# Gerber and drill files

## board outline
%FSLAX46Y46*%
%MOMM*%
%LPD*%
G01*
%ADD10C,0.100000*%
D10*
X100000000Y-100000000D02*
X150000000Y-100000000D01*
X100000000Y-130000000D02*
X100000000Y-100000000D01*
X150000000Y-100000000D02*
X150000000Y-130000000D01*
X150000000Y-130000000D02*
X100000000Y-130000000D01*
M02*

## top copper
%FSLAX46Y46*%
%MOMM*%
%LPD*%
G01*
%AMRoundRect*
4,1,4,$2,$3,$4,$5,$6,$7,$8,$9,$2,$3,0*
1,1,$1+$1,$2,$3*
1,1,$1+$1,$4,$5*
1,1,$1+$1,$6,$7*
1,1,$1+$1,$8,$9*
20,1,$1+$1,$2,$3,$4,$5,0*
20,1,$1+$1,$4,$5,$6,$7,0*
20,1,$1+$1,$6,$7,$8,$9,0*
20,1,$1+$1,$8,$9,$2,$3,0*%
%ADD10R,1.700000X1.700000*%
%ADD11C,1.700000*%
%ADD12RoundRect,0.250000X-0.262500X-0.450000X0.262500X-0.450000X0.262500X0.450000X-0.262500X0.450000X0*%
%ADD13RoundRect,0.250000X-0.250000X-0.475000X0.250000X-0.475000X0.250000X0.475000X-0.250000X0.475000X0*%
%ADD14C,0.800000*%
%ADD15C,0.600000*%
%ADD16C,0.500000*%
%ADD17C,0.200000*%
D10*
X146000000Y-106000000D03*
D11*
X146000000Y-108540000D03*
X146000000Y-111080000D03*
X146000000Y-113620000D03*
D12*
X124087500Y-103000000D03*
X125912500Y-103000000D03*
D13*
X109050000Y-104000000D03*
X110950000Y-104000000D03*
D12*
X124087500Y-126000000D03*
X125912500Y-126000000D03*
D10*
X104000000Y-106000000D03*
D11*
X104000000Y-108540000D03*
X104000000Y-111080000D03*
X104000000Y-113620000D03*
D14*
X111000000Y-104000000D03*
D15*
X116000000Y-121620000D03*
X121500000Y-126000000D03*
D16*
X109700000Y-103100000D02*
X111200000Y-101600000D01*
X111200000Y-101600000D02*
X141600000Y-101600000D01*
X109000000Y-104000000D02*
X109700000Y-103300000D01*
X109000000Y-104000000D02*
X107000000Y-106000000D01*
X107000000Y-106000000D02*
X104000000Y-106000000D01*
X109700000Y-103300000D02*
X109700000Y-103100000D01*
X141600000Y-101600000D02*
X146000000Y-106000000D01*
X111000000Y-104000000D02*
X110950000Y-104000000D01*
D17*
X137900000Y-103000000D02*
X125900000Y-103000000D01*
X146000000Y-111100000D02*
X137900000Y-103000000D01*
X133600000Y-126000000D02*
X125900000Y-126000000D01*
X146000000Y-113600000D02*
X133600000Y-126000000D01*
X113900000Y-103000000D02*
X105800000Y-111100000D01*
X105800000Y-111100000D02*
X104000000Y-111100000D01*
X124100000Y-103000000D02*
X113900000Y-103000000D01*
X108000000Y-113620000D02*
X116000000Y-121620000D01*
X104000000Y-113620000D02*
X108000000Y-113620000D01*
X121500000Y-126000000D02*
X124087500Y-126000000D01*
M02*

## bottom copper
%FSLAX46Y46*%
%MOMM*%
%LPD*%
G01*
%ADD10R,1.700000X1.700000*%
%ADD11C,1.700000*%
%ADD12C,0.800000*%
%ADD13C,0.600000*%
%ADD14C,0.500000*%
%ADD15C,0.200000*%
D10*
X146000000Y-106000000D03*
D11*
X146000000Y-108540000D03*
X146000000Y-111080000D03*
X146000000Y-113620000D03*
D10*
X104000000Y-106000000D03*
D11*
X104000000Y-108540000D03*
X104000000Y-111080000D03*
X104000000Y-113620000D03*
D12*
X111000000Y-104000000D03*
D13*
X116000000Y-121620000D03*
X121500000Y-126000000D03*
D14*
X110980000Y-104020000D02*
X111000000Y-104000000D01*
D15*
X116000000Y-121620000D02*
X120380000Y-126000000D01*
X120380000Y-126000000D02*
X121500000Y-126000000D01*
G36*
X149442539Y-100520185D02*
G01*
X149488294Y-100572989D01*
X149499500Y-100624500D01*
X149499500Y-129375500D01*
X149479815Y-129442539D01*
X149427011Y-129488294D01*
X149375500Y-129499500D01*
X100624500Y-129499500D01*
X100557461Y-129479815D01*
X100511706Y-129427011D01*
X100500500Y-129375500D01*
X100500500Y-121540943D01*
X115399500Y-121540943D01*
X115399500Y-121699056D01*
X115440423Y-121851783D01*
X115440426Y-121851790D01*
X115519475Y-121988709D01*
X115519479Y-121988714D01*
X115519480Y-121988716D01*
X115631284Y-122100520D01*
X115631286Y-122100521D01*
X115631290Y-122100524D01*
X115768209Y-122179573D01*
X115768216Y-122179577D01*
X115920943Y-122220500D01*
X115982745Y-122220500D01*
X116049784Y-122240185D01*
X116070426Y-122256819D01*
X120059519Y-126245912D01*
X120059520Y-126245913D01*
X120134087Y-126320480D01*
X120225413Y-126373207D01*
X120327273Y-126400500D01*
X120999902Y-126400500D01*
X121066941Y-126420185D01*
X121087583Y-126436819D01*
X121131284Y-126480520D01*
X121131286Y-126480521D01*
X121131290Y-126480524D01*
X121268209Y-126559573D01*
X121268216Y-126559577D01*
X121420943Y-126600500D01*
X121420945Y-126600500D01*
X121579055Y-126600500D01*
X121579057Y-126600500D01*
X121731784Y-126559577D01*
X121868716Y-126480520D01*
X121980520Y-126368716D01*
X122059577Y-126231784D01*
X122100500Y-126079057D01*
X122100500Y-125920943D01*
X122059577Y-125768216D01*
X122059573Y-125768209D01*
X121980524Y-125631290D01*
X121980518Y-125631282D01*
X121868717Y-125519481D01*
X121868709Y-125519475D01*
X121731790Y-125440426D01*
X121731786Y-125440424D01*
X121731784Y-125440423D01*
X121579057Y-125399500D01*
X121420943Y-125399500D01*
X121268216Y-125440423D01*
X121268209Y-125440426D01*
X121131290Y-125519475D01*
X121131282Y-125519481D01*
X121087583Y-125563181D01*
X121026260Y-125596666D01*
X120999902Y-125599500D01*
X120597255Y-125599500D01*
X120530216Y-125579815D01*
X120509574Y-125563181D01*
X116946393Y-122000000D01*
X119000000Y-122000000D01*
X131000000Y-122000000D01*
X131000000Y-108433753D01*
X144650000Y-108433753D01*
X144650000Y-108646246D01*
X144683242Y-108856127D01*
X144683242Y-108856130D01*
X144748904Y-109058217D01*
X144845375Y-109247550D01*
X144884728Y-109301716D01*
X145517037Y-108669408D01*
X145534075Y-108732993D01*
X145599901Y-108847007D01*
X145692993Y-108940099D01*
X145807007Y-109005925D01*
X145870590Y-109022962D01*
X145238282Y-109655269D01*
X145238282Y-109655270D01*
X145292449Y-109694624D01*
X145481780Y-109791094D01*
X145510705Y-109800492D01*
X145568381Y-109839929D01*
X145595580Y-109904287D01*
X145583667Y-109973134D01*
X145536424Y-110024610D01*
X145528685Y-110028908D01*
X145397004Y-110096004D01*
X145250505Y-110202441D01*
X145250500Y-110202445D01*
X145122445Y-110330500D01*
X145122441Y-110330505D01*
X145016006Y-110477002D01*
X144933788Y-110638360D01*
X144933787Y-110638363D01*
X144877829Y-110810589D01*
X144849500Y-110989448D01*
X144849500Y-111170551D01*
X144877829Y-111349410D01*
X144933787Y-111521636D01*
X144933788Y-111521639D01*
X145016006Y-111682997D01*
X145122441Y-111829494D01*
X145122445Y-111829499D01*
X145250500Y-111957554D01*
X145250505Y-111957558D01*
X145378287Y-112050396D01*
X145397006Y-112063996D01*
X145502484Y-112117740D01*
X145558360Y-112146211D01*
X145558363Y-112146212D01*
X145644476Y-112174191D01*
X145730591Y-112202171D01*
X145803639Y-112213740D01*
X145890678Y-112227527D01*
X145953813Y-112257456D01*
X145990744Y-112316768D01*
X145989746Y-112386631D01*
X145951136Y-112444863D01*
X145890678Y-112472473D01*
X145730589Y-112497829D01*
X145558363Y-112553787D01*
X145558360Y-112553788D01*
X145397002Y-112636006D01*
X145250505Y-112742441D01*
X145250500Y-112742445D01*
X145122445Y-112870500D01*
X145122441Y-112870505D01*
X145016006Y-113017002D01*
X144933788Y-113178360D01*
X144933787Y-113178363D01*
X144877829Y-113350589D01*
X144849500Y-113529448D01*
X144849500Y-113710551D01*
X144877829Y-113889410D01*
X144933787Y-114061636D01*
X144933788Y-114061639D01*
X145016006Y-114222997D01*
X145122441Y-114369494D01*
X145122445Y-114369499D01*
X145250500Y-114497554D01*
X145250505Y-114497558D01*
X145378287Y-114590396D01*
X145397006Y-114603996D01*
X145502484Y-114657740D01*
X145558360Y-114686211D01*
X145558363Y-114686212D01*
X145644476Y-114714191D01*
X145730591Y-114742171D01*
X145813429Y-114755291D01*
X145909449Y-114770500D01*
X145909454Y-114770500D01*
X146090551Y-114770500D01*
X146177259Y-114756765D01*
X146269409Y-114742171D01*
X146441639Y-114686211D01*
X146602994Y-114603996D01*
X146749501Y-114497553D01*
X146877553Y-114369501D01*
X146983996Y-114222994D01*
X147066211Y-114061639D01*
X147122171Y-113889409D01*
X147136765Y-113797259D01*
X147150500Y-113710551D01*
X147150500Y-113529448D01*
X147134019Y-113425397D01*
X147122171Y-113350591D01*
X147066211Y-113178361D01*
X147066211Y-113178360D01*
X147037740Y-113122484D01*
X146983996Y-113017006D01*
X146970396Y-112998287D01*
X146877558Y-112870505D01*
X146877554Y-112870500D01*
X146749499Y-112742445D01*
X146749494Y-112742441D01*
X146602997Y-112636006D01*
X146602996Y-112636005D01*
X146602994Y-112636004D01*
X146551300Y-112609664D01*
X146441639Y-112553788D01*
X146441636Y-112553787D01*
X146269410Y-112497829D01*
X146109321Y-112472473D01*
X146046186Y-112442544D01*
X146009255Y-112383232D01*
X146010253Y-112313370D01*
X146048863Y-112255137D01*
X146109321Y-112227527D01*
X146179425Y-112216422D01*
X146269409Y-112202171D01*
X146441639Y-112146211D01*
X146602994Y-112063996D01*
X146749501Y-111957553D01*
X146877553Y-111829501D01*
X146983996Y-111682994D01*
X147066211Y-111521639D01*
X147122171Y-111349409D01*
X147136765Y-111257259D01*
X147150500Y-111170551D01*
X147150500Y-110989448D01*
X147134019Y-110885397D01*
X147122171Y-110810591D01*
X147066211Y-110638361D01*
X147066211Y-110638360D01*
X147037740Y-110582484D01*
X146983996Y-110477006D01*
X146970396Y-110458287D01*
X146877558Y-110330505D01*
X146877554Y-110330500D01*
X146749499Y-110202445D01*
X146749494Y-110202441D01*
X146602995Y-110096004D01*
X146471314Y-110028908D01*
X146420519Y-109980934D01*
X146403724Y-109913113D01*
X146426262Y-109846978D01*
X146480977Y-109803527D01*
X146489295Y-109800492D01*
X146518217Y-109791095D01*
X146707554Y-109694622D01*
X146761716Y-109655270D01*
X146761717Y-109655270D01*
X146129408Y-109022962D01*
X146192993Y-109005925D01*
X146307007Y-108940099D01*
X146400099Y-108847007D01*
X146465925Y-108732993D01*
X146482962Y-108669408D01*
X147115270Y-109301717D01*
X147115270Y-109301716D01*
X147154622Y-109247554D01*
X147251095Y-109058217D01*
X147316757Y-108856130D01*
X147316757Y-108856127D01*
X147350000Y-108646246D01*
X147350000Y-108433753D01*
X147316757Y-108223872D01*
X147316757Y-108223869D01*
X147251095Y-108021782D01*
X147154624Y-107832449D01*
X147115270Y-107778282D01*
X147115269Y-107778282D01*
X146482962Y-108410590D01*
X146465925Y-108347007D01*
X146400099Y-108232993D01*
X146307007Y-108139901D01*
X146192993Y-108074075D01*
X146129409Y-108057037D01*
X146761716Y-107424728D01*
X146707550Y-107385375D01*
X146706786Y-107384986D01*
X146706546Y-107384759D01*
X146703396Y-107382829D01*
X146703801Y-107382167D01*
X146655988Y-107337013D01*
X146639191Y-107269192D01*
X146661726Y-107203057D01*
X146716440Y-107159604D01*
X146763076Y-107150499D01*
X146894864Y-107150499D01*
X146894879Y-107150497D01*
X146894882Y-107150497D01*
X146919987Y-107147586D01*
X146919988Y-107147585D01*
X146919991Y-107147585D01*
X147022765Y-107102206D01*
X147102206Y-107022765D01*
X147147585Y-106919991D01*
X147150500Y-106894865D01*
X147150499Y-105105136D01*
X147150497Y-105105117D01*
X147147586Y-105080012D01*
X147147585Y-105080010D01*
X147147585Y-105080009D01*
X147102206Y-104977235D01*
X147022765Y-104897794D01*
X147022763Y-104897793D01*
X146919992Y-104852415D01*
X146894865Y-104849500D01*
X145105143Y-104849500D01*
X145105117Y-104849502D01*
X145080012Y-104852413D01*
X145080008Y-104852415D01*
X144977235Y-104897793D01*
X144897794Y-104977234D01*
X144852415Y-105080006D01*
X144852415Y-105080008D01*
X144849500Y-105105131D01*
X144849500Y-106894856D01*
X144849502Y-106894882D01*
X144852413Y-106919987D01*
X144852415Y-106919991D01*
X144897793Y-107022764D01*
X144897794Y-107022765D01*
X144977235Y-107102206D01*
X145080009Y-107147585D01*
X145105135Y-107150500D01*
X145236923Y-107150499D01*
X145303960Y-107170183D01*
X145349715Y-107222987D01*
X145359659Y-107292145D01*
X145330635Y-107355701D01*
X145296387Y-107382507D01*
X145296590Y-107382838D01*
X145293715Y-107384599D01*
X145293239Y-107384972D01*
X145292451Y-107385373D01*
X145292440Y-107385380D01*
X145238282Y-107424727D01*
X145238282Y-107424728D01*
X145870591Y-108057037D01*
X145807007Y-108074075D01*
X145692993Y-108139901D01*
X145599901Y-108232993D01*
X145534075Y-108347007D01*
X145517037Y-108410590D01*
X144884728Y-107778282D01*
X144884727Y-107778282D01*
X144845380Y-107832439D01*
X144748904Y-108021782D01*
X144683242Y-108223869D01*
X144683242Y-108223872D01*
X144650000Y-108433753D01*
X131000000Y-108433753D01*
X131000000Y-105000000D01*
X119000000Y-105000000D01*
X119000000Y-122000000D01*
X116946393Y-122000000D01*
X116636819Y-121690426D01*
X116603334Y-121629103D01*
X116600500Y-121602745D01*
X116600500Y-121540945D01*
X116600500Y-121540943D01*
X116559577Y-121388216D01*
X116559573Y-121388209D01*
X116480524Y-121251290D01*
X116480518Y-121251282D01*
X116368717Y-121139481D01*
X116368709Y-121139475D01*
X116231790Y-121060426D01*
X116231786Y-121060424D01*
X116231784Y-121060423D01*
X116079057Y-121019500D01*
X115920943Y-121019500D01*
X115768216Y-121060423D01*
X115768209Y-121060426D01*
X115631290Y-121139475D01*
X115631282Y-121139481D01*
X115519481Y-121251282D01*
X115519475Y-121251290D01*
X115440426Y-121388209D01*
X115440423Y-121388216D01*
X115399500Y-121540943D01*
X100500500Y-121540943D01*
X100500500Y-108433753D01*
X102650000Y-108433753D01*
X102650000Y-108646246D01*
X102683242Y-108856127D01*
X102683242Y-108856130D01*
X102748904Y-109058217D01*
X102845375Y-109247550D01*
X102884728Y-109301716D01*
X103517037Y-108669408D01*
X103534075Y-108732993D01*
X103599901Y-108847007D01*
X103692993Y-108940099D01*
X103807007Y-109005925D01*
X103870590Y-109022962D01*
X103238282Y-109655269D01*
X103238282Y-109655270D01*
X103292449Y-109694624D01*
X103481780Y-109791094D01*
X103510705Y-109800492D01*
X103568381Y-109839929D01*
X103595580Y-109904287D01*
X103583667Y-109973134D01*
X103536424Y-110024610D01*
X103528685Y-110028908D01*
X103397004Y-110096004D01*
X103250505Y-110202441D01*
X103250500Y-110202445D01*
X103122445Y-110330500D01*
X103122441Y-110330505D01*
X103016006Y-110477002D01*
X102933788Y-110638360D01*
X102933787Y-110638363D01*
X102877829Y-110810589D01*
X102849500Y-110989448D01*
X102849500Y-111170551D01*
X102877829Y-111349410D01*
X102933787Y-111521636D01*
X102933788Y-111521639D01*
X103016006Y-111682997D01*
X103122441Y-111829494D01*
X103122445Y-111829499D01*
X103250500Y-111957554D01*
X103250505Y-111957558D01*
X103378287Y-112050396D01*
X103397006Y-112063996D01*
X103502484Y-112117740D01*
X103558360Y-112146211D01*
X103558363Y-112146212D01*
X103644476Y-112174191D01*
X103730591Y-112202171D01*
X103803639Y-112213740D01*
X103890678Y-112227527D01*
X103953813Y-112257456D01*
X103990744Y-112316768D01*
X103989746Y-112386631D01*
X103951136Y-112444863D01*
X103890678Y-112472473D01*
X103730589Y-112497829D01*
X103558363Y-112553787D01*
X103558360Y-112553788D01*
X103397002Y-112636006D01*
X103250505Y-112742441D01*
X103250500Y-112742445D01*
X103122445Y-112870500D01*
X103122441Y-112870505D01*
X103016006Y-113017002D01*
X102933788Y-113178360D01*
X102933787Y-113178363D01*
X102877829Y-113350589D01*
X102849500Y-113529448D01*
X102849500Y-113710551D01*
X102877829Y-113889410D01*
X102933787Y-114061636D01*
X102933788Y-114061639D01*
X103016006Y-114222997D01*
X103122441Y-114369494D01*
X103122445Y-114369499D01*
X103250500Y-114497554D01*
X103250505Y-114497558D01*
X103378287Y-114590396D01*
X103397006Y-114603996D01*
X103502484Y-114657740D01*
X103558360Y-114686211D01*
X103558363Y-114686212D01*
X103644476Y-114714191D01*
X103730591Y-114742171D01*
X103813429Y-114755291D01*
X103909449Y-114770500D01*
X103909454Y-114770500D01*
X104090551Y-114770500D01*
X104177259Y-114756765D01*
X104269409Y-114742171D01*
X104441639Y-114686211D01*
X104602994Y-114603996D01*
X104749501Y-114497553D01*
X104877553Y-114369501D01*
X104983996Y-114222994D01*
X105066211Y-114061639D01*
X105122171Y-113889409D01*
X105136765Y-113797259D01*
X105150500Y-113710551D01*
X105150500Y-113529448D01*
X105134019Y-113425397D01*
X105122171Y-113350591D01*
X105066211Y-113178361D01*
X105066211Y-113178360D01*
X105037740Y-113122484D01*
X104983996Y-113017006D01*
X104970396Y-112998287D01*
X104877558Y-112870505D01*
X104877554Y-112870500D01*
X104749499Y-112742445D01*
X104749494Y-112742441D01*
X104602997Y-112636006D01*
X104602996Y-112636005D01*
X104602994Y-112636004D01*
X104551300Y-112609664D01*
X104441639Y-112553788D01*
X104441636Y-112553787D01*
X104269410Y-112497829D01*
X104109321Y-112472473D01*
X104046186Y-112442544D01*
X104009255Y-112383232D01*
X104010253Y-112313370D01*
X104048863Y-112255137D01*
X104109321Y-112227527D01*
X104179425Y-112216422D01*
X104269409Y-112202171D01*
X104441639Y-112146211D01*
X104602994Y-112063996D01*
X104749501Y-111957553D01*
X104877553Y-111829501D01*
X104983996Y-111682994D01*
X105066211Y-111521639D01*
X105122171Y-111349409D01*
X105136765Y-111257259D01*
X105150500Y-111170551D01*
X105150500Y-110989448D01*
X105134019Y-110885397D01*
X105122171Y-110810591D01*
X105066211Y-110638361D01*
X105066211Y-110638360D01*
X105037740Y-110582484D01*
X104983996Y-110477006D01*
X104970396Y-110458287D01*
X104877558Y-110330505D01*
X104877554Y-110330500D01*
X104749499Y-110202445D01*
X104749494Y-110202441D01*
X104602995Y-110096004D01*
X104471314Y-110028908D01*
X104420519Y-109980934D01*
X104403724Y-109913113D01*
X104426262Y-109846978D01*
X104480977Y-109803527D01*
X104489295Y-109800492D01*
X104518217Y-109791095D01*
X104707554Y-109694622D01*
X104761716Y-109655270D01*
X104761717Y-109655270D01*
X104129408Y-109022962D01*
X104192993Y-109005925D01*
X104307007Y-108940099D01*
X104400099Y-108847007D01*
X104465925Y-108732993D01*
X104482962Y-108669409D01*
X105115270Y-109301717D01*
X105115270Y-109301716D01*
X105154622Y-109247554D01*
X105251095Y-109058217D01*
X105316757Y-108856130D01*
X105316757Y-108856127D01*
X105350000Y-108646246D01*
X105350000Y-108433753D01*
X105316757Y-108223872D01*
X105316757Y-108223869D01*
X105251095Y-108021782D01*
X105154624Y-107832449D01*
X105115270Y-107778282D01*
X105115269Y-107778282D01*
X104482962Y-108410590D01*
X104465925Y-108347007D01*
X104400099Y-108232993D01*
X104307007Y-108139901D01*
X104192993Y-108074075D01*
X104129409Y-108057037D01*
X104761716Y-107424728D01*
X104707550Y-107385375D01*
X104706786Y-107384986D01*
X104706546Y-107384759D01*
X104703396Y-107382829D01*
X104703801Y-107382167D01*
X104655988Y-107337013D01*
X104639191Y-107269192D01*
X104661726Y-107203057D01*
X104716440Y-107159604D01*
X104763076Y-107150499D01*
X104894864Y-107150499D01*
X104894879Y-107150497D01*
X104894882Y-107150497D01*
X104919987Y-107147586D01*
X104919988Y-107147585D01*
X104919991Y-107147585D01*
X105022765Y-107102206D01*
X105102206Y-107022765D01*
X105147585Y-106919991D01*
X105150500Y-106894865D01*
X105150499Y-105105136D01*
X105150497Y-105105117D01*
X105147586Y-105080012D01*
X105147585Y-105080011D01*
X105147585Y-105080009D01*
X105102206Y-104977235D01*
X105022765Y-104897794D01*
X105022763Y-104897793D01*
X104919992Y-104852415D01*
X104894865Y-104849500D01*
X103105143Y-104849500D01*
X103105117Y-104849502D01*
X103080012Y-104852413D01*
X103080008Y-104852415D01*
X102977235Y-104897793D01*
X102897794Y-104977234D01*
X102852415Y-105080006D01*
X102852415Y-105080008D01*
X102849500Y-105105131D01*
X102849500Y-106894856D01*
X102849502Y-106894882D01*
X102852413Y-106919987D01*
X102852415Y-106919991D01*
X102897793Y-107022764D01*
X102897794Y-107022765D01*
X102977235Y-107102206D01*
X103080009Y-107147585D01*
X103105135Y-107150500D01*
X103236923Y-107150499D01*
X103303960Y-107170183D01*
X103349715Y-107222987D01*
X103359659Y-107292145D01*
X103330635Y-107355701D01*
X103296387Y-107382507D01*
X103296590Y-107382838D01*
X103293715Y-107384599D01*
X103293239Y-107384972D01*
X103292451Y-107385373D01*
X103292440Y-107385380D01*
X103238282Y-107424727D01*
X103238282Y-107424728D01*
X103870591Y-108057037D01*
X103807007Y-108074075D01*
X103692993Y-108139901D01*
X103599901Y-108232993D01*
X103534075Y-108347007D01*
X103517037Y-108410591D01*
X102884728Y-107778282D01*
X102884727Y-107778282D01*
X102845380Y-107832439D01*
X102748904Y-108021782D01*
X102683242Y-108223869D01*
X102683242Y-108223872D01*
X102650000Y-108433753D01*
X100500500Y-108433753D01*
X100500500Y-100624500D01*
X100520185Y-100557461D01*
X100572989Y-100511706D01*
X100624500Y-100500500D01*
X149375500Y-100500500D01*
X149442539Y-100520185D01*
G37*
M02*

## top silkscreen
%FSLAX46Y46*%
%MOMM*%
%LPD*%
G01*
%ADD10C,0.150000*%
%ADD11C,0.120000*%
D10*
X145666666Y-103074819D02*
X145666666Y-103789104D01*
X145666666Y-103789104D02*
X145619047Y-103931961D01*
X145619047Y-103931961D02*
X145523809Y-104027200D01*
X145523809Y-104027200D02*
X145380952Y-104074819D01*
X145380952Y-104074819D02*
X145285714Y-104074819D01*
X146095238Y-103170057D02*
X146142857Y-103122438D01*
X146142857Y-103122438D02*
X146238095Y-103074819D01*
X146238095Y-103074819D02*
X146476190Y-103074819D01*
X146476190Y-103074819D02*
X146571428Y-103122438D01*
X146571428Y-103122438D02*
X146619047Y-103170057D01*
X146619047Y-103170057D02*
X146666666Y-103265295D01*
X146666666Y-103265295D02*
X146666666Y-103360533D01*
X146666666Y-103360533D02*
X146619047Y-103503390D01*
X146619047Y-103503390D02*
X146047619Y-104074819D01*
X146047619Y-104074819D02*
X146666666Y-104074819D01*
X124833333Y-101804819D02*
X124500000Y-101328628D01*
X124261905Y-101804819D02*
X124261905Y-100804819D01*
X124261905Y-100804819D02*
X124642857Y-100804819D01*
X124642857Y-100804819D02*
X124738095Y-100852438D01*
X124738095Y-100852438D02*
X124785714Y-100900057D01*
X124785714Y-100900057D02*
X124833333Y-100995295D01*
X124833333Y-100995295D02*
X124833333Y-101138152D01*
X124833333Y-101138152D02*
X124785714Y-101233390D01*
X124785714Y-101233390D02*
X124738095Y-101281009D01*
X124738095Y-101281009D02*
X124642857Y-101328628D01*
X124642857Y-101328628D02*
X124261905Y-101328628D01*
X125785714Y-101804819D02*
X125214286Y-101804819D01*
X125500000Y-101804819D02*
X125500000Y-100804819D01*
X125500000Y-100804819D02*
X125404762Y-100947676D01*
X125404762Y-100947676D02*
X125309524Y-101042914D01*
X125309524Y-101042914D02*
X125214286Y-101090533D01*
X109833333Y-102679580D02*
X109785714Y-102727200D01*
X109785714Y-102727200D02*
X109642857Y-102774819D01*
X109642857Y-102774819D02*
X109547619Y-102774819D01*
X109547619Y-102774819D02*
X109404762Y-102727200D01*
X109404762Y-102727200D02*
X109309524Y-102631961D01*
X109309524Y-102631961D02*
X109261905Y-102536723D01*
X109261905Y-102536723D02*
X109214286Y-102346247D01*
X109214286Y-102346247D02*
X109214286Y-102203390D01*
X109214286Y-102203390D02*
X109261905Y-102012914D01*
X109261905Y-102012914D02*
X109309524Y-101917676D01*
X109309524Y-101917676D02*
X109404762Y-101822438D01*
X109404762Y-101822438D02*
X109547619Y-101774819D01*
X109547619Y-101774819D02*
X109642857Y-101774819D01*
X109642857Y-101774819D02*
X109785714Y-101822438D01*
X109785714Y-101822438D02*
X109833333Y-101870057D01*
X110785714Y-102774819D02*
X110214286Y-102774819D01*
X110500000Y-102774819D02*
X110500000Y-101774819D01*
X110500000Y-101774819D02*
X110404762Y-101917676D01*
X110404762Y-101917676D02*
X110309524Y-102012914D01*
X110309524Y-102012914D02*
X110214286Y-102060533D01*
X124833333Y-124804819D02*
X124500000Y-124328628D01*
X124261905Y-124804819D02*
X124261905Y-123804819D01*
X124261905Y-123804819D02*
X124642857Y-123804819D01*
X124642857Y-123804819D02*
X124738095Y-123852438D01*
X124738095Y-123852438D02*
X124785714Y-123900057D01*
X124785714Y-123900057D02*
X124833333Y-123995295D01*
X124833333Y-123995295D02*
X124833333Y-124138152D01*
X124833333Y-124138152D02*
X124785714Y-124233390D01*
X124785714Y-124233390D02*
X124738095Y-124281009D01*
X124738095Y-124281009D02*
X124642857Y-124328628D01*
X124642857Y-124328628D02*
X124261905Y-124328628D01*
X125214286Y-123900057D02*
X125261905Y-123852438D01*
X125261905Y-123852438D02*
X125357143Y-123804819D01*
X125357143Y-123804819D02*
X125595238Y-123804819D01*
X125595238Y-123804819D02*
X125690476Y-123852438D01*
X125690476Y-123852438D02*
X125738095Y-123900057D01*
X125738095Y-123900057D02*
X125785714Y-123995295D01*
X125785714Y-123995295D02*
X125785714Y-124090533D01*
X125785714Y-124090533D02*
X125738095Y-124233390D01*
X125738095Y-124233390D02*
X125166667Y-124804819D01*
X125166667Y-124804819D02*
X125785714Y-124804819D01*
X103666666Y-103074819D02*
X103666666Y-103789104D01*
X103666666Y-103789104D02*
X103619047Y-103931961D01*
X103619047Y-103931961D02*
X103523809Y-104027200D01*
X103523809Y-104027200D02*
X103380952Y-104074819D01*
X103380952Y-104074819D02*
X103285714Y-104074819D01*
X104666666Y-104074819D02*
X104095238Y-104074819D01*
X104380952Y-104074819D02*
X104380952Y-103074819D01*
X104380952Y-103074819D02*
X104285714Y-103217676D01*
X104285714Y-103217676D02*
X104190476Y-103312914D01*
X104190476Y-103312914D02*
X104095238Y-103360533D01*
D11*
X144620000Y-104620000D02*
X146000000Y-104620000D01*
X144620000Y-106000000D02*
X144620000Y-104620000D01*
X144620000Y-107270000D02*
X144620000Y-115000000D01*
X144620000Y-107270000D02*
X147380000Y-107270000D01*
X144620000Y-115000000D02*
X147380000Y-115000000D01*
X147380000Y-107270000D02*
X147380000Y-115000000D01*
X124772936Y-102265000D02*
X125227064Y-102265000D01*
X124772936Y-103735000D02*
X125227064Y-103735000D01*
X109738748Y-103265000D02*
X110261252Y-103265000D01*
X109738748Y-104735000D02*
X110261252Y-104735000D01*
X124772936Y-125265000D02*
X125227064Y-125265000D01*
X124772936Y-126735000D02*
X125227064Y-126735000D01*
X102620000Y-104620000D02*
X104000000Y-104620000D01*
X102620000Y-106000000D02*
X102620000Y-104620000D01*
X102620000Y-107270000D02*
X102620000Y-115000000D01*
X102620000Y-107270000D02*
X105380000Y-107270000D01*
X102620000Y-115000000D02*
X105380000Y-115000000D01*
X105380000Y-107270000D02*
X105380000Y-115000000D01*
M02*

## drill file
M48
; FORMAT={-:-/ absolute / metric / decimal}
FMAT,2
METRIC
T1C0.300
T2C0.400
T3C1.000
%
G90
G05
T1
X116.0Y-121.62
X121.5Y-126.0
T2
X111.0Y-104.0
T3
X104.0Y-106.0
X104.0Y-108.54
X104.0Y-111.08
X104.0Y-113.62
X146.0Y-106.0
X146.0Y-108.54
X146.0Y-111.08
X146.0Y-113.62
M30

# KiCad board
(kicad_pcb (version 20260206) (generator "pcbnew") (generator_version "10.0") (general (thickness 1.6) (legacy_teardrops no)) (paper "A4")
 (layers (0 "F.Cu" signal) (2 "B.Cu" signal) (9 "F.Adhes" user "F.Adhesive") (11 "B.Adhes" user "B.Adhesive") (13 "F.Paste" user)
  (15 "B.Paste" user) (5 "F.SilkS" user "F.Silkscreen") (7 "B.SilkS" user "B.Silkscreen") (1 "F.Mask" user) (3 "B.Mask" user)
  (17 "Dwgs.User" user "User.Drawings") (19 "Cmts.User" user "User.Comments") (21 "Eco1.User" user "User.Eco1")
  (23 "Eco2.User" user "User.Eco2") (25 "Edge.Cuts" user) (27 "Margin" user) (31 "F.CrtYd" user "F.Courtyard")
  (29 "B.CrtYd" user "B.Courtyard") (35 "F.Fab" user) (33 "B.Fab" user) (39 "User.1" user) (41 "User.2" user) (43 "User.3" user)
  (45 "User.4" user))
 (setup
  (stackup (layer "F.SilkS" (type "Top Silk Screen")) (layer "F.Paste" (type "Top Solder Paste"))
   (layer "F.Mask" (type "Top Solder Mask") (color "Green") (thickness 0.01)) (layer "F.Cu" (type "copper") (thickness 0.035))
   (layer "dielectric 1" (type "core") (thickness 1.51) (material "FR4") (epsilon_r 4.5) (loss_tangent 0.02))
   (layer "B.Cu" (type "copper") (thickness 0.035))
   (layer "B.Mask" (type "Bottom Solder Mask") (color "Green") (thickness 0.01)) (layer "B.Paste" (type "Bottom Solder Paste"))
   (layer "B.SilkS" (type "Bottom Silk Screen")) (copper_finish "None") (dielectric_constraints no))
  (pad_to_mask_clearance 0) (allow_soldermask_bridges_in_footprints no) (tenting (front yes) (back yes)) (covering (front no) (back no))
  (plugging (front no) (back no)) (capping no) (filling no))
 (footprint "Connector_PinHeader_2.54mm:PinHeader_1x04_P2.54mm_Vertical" (layer "F.Cu") (at 146 106)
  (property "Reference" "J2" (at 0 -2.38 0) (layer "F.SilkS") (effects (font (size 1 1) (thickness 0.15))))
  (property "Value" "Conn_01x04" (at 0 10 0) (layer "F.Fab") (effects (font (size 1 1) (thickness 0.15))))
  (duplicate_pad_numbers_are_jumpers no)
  (fp_line (start -1.38 -1.38) (end 0 -1.38) (stroke (width 0.12) (type solid)) (layer "F.SilkS"))
  (fp_line (start -1.38 0) (end -1.38 -1.38) (stroke (width 0.12) (type solid)) (layer "F.SilkS"))
  (fp_line (start -1.38 1.27) (end -1.38 9) (stroke (width 0.12) (type solid)) (layer "F.SilkS"))
  (fp_line (start -1.38 1.27) (end 1.38 1.27) (stroke (width 0.12) (type solid)) (layer "F.SilkS"))
  (fp_line (start -1.38 9) (end 1.38 9) (stroke (width 0.12) (type solid)) (layer "F.SilkS"))
  (fp_line (start 1.38 1.27) (end 1.38 9) (stroke (width 0.12) (type solid)) (layer "F.SilkS"))
  (pad "1" thru_hole rect (at 0 0) (size 1.7 1.7) (drill 1) (layers "*.Cu" "*.Mask") (remove_unused_layers no) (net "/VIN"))
  (pad "2" thru_hole circle (at 0 2.54) (size 1.7 1.7) (drill 1) (layers "*.Cu" "*.Mask") (remove_unused_layers no) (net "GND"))
  (pad "3" thru_hole circle (at 0 5.08) (size 1.7 1.7) (drill 1) (layers "*.Cu" "*.Mask") (remove_unused_layers no) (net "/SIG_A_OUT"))
  (pad "4" thru_hole circle (at 0 7.62) (size 1.7 1.7) (drill 1) (layers "*.Cu" "*.Mask") (remove_unused_layers no) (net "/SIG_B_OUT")))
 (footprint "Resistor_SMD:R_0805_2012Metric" (layer "F.Cu") (at 125 103)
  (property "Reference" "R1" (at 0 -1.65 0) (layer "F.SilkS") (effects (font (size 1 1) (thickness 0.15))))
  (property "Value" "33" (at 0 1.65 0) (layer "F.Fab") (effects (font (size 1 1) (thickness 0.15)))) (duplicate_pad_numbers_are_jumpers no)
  (fp_line (start -0.227064 -0.735) (end 0.227064 -0.735) (stroke (width 0.12) (type solid)) (layer "F.SilkS"))
  (fp_line (start -0.227064 0.735) (end 0.227064 0.735) (stroke (width 0.12) (type solid)) (layer "F.SilkS"))
  (pad "1" smd roundrect (at -0.9125 0) (size 1.025 1.4) (layers "F.Cu" "F.Mask" "F.Paste") (roundrect_rratio 0.243902) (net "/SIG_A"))
  (pad "2" smd roundrect (at 0.9125 0) (size 1.025 1.4) (layers "F.Cu" "F.Mask" "F.Paste") (roundrect_rratio 0.243902) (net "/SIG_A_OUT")))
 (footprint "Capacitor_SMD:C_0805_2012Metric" (layer "F.Cu") (at 110 104)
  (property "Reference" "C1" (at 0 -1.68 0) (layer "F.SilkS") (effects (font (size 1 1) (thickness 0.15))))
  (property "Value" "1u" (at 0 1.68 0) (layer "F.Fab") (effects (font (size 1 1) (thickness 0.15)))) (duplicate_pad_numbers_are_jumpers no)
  (fp_line (start -0.261252 -0.735) (end 0.261252 -0.735) (stroke (width 0.12) (type solid)) (layer "F.SilkS"))
  (fp_line (start -0.261252 0.735) (end 0.261252 0.735) (stroke (width 0.12) (type solid)) (layer "F.SilkS"))
  (pad "1" smd roundrect (at -0.95 0) (size 1 1.45) (layers "F.Cu" "F.Mask" "F.Paste") (roundrect_rratio 0.25) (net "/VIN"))
  (pad "2" smd roundrect (at 0.95 0) (size 1 1.45) (layers "F.Cu" "F.Mask" "F.Paste") (roundrect_rratio 0.25) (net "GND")))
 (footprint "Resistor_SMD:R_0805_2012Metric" (layer "F.Cu") (at 125 126)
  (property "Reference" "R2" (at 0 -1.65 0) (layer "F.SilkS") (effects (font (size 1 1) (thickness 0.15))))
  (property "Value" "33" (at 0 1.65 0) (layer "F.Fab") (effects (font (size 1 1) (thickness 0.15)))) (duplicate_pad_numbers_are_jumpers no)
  (fp_line (start -0.227064 -0.735) (end 0.227064 -0.735) (stroke (width 0.12) (type solid)) (layer "F.SilkS"))
  (fp_line (start -0.227064 0.735) (end 0.227064 0.735) (stroke (width 0.12) (type solid)) (layer "F.SilkS"))
  (pad "1" smd roundrect (at -0.9125 0) (size 1.025 1.4) (layers "F.Cu" "F.Mask" "F.Paste") (roundrect_rratio 0.243902) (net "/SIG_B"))
  (pad "2" smd roundrect (at 0.9125 0) (size 1.025 1.4) (layers "F.Cu" "F.Mask" "F.Paste") (roundrect_rratio 0.243902) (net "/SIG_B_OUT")))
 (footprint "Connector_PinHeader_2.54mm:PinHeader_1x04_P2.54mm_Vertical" (layer "F.Cu") (at 104 106)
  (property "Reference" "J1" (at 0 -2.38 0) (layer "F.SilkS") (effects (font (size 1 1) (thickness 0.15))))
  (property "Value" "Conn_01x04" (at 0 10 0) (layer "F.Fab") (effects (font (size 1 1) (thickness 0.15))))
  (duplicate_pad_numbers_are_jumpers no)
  (fp_line (start -1.38 -1.38) (end 0 -1.38) (stroke (width 0.12) (type solid)) (layer "F.SilkS"))
  (fp_line (start -1.38 0) (end -1.38 -1.38) (stroke (width 0.12) (type solid)) (layer "F.SilkS"))
  (fp_line (start -1.38 1.27) (end -1.38 9) (stroke (width 0.12) (type solid)) (layer "F.SilkS"))
  (fp_line (start -1.38 1.27) (end 1.38 1.27) (stroke (width 0.12) (type solid)) (layer "F.SilkS"))
  (fp_line (start -1.38 9) (end 1.38 9) (stroke (width 0.12) (type solid)) (layer "F.SilkS"))
  (fp_line (start 1.38 1.27) (end 1.38 9) (stroke (width 0.12) (type solid)) (layer "F.SilkS"))
  (pad "1" thru_hole rect (at 0 0) (size 1.7 1.7) (drill 1) (layers "*.Cu" "*.Mask") (remove_unused_layers no) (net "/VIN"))
  (pad "2" thru_hole circle (at 0 2.54) (size 1.7 1.7) (drill 1) (layers "*.Cu" "*.Mask") (remove_unused_layers no) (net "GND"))
  (pad "3" thru_hole circle (at 0 5.08) (size 1.7 1.7) (drill 1) (layers "*.Cu" "*.Mask") (remove_unused_layers no) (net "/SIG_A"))
  (pad "4" thru_hole circle (at 0 7.62) (size 1.7 1.7) (drill 1) (layers "*.Cu" "*.Mask") (remove_unused_layers no) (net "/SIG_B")))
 (gr_line (start 100 100) (end 150 100) (stroke (width 0.1) (type default)) (layer "Edge.Cuts"))
 (gr_line (start 100 130) (end 100 100) (stroke (width 0.1) (type default)) (layer "Edge.Cuts"))
 (gr_line (start 150 100) (end 150 130) (stroke (width 0.1) (type default)) (layer "Edge.Cuts"))
 (gr_line (start 150 130) (end 100 130) (stroke (width 0.1) (type default)) (layer "Edge.Cuts"))
 (segment (start 109.7 103.1) (end 111.2 101.6) (width 0.5) (layer "F.Cu") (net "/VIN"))
 (segment (start 111.2 101.6) (end 141.6 101.6) (width 0.5) (layer "F.Cu") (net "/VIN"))
 (segment (start 109 104) (end 109.7 103.3) (width 0.5) (layer "F.Cu") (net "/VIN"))
 (segment (start 109 104) (end 107 106) (width 0.5) (layer "F.Cu") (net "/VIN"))
 (segment (start 107 106) (end 104 106) (width 0.5) (layer "F.Cu") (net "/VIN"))
 (segment (start 109.7 103.3) (end 109.7 103.1) (width 0.5) (layer "F.Cu") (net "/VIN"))
 (segment (start 141.6 101.6) (end 146 106) (width 0.5) (layer "F.Cu") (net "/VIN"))
 (segment (start 111 104) (end 110.95 104) (width 0.5) (layer "F.Cu") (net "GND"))
 (via (at 111 104) (size 0.8) (drill 0.4) (layers "F.Cu" "B.Cu") (capping yes) (filling yes) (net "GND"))
 (segment (start 110.98 104.02) (end 111 104) (width 0.5) (layer "B.Cu") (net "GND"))
 (segment (start 137.9 103) (end 125.9 103) (width 0.2) (layer "F.Cu") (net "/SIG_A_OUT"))
 (segment (start 146 111.1) (end 137.9 103) (width 0.2) (layer "F.Cu") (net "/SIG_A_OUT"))
 (segment (start 133.6 126) (end 125.9 126) (width 0.2) (layer "F.Cu") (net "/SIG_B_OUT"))
 (segment (start 146 113.6) (end 133.6 126) (width 0.2) (layer "F.Cu") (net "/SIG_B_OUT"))
 (segment (start 113.9 103) (end 105.8 111.1) (width 0.2) (layer "F.Cu") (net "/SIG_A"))
 (segment (start 105.8 111.1) (end 104 111.1) (width 0.2) (layer "F.Cu") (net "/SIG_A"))
 (segment (start 124.1 103) (end 113.9 103) (width 0.2) (layer "F.Cu") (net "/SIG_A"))
 (segment (start 108 113.62) (end 116 121.62) (width 0.2) (locked yes) (layer "F.Cu") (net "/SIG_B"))
 (segment (start 104 113.62) (end 108 113.62) (width 0.2) (locked yes) (layer "F.Cu") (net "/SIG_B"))
 (segment (start 121.5 126) (end 124.0875 126) (width 0.2) (locked yes) (layer "F.Cu") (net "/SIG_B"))
 (via (at 116 121.62) (size 0.6) (drill 0.3) (layers "F.Cu" "B.Cu") (locked yes) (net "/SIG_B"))
 (via (at 121.5 126) (size 0.6) (drill 0.3) (layers "F.Cu" "B.Cu") (locked yes) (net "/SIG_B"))
 (segment (start 116 121.62) (end 120.38 126) (width 0.2) (locked yes) (layer "B.Cu") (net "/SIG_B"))
 (segment (start 120.38 126) (end 121.5 126) (width 0.2) (locked yes) (layer "B.Cu") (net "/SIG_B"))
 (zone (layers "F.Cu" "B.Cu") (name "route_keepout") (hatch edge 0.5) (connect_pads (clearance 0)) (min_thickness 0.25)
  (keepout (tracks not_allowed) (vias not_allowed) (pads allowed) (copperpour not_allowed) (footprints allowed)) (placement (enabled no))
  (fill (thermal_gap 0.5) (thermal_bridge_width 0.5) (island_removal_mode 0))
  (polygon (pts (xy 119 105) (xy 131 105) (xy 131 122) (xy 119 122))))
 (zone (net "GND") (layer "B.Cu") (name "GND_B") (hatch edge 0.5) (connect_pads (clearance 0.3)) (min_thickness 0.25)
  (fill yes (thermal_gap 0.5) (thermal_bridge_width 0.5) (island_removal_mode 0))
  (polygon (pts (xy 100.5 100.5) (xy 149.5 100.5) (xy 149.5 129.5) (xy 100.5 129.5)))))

